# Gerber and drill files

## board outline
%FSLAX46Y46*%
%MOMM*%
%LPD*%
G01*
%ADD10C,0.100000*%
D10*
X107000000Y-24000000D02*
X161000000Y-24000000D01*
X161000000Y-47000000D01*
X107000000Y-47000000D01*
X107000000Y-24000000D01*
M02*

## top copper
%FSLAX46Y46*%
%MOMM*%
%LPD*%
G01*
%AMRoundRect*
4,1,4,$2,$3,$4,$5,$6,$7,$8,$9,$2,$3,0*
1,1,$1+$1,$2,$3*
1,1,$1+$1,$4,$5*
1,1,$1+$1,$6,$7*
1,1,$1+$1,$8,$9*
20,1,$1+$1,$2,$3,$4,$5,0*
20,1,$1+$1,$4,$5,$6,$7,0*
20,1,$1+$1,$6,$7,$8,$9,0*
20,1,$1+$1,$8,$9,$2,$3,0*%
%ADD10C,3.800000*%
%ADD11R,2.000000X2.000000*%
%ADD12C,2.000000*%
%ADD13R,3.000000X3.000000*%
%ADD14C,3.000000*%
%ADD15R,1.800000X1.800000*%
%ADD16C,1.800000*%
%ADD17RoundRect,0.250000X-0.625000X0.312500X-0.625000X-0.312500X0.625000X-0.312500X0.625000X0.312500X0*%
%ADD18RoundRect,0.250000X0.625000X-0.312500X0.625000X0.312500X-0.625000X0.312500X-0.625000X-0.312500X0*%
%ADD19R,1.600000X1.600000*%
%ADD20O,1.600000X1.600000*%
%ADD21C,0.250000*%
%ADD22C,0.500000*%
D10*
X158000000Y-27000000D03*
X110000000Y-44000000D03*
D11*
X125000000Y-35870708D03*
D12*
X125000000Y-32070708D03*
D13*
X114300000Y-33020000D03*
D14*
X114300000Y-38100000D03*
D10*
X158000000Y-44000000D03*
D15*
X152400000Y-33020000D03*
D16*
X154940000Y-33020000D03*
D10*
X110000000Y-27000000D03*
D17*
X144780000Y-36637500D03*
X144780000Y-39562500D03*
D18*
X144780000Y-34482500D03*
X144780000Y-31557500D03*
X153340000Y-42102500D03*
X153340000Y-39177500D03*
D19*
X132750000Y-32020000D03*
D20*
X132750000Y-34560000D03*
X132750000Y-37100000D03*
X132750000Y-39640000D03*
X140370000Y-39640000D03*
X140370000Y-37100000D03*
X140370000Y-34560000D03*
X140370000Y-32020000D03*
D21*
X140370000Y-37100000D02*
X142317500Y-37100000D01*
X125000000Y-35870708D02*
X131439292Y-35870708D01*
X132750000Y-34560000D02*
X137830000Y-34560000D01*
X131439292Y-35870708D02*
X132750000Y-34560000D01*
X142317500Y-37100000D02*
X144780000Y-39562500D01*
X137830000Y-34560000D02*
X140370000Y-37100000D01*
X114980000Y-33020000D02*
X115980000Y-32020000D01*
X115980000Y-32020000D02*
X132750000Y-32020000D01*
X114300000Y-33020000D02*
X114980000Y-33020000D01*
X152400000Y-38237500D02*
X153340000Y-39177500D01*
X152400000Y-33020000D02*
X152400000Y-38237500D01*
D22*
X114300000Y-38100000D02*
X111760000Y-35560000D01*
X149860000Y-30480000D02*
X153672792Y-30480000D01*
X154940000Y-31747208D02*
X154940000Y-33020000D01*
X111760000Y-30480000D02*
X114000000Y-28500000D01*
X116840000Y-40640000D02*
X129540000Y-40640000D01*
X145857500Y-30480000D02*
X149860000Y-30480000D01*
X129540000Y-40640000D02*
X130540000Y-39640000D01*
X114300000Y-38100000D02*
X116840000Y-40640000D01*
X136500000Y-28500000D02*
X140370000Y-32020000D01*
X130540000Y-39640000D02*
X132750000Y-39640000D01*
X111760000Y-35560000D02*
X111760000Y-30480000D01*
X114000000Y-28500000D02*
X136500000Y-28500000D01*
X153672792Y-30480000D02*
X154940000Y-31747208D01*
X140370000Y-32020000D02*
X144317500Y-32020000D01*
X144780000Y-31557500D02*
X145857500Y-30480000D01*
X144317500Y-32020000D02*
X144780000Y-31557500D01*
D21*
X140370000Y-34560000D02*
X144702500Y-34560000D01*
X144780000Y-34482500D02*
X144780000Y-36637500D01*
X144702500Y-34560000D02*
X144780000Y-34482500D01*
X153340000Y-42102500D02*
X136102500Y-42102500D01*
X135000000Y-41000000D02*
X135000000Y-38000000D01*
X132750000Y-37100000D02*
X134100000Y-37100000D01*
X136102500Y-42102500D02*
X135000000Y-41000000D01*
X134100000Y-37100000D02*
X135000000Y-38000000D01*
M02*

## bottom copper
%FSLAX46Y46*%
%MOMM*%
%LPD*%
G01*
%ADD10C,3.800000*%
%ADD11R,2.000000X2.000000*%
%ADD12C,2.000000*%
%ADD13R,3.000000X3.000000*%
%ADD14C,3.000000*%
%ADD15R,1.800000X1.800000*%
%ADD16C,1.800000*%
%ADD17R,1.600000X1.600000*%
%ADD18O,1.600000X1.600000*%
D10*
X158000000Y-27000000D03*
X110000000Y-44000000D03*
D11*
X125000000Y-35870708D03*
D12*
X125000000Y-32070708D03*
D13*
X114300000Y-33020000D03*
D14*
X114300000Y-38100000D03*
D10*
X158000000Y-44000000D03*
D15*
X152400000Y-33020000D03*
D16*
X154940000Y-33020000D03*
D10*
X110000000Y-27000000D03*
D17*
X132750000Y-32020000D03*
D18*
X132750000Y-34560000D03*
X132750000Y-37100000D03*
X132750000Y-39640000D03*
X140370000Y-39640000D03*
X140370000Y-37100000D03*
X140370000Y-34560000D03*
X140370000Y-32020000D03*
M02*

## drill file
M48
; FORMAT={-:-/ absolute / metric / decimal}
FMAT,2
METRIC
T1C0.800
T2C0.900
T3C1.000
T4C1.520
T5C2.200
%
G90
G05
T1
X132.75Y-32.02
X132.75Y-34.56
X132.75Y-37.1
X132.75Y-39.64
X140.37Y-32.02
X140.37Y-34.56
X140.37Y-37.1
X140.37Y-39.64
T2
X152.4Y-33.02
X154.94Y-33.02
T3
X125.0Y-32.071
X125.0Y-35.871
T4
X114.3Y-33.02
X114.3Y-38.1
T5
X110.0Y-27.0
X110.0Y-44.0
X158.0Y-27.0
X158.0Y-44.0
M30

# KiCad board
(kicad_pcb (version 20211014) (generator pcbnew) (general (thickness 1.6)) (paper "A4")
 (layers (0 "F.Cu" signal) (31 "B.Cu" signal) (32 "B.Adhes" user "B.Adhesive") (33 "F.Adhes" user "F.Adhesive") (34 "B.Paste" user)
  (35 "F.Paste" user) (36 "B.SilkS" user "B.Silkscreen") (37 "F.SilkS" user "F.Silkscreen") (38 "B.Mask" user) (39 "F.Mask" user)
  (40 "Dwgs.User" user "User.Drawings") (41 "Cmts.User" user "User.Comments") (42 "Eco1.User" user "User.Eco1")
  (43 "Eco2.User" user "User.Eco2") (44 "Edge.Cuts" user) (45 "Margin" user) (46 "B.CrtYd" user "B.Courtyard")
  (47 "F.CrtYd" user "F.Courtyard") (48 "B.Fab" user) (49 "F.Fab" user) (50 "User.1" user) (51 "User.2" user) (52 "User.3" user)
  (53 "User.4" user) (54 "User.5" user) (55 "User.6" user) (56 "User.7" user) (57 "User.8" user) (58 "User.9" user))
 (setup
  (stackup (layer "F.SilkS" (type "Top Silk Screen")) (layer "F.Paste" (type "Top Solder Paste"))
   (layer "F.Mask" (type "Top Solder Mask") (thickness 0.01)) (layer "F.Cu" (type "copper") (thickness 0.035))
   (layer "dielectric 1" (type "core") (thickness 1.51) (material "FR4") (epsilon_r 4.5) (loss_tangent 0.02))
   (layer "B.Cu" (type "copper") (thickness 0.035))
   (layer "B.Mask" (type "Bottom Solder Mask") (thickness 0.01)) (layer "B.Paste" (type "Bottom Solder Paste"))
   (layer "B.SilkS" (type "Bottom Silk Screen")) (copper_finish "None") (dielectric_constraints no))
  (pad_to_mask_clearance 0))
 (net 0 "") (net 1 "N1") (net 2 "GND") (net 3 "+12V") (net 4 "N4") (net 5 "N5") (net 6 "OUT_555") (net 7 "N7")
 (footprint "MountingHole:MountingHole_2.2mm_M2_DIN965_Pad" (layer "F.Cu") (at 158 27)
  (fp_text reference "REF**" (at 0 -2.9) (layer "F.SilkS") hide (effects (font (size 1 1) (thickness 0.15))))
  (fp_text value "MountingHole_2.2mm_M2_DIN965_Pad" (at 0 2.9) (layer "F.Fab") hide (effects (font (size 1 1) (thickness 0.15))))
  (pad "1" thru_hole circle (at 0 0) (size 3.8 3.8) (drill 2.2) (layers *.Cu *.Mask)))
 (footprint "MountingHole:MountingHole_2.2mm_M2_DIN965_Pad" (layer "F.Cu") (at 110 44)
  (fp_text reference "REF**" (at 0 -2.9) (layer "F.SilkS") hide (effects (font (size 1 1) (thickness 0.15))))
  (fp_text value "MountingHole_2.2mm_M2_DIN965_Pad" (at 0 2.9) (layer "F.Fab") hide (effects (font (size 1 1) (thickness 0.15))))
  (pad "1" thru_hole circle (at 0 0) (size 3.8 3.8) (drill 2.2) (layers *.Cu *.Mask)))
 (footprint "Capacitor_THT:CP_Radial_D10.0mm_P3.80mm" (layer "F.Cu") (at 125 35.870708 90)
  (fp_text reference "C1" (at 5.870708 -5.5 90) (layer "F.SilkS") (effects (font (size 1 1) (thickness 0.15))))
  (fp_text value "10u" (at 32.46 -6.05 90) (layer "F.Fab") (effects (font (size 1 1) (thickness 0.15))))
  (pad "1" thru_hole rect (at 0 0 90) (size 2 2) (drill 1) (layers *.Cu *.Mask) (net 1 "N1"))
  (pad "2" thru_hole circle (at 3.8 0 90) (size 2 2) (drill 1) (layers *.Cu *.Mask) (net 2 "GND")))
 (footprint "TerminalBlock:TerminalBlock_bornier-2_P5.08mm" (layer "F.Cu") (at 114.3 33.02 -90)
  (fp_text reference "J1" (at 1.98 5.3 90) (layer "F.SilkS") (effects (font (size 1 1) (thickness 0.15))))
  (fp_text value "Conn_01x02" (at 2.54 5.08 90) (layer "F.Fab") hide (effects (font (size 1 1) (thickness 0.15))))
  (pad "1" thru_hole rect (at 0 0 270) (size 3 3) (drill 1.52) (layers *.Cu *.Mask) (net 2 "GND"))
  (pad "2" thru_hole circle (at 5.08 0 270) (size 3 3) (drill 1.52) (layers *.Cu *.Mask) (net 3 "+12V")))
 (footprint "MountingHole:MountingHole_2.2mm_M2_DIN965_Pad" (layer "F.Cu") (at 158 44)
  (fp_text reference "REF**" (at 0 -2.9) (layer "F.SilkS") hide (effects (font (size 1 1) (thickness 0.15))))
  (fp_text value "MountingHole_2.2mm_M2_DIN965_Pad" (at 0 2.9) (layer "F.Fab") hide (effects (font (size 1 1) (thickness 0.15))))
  (pad "1" thru_hole circle (at 0 0) (size 3.8 3.8) (drill 2.2) (layers *.Cu *.Mask)))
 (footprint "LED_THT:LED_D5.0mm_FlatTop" (layer "F.Cu") (at 152.4 33.02)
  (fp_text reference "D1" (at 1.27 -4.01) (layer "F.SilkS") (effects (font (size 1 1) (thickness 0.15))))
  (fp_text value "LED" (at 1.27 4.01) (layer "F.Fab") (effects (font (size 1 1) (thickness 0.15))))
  (pad "1" thru_hole rect locked (at 0 0) (size 1.8 1.8) (drill 0.9) (layers *.Cu *.Mask) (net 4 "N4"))
  (pad "2" thru_hole circle (at 2.54 0) (size 1.8 1.8) (drill 0.9) (layers *.Cu *.Mask) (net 3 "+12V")))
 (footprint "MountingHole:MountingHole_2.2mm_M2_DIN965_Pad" (layer "F.Cu") (at 110 27)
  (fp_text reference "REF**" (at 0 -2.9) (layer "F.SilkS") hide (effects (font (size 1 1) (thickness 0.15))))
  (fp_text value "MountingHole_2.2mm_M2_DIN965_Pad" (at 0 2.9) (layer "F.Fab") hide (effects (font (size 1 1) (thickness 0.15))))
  (pad "1" thru_hole circle (at 0 0) (size 3.8 3.8) (drill 2.2) (layers *.Cu *.Mask)))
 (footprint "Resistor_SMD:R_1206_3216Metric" (layer "F.Cu") (at 144.78 38.1 -90)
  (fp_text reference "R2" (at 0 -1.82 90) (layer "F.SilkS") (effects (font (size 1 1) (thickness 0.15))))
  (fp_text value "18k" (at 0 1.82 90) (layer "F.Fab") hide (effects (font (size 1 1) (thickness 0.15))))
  (pad "1" smd roundrect (at -1.4625 0 270) (size 1.125 1.75) (layers "F.Cu" "F.Paste" "F.Mask") (roundrect_rratio 0.222222) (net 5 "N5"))
  (pad "2" smd roundrect (at 1.4625 0 270) (size 1.125 1.75) (layers "F.Cu" "F.Paste" "F.Mask") (roundrect_rratio 0.222222) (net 1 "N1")))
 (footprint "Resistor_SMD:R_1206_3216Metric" (layer "F.Cu") (at 144.78 33.02 90)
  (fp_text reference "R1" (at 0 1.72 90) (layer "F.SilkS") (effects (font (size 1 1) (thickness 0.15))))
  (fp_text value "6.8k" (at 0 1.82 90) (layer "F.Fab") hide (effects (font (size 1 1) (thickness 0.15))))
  (pad "1" smd roundrect (at -1.4625 0 90) (size 1.125 1.75) (layers "F.Cu" "F.Paste" "F.Mask") (roundrect_rratio 0.222222) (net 5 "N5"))
  (pad "2" smd roundrect (at 1.4625 0 90) (size 1.125 1.75) (layers "F.Cu" "F.Paste" "F.Mask") (roundrect_rratio 0.222222) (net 3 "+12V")))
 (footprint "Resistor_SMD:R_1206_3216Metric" (layer "F.Cu") (at 153.34 40.64 90)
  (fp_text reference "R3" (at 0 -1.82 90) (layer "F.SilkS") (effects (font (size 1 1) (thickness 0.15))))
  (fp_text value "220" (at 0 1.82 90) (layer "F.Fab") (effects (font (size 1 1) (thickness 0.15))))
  (pad "1" smd roundrect (at -1.4625 0 90) (size 1.125 1.75) (layers "F.Cu" "F.Paste" "F.Mask") (roundrect_rratio 0.222222)
   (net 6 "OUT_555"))
  (pad "2" smd roundrect (at 1.4625 0 90) (size 1.125 1.75) (layers "F.Cu" "F.Paste" "F.Mask") (roundrect_rratio 0.222222) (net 4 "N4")))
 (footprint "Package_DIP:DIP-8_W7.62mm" (layer "F.Cu") (at 132.75 32.02)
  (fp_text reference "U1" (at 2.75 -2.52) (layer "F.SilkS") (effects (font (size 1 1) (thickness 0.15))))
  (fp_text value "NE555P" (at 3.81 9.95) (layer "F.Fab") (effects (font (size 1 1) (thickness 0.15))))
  (pad "1" thru_hole rect (at 0 0) (size 1.6 1.6) (drill 0.8) (layers *.Cu *.Mask) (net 2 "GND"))
  (pad "2" thru_hole oval (at 0 2.54) (size 1.6 1.6) (drill 0.8) (layers *.Cu *.Mask) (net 1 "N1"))
  (pad "3" thru_hole oval (at 0 5.08) (size 1.6 1.6) (drill 0.8) (layers *.Cu *.Mask) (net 6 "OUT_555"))
  (pad "4" thru_hole oval (at 0 7.62) (size 1.6 1.6) (drill 0.8) (layers *.Cu *.Mask) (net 3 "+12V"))
  (pad "5" thru_hole oval (at 7.62 7.62) (size 1.6 1.6) (drill 0.8) (layers *.Cu *.Mask) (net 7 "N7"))
  (pad "6" thru_hole oval (at 7.62 5.08) (size 1.6 1.6) (drill 0.8) (layers *.Cu *.Mask) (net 1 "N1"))
  (pad "7" thru_hole oval (at 7.62 2.54) (size 1.6 1.6) (drill 0.8) (layers *.Cu *.Mask) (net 5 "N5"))
  (pad "8" thru_hole oval (at 7.62 0) (size 1.6 1.6) (drill 0.8) (layers *.Cu *.Mask) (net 3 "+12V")))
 (gr_rect (start 107 24) (end 161 47) (layer "Edge.Cuts") (width 0.1) (fill none))
 (segment (start 140.37 37.1) (end 142.3175 37.1) (width 0.25) (layer "F.Cu") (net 1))
 (segment (start 125 35.870708) (end 131.439292 35.870708) (width 0.25) (layer "F.Cu") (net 1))
 (segment (start 132.75 34.56) (end 137.83 34.56) (width 0.25) (layer "F.Cu") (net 1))
 (segment (start 131.439292 35.870708) (end 132.75 34.56) (width 0.25) (layer "F.Cu") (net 1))
 (segment (start 142.3175 37.1) (end 144.78 39.5625) (width 0.25) (layer "F.Cu") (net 1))
 (segment (start 137.83 34.56) (end 140.37 37.1) (width 0.25) (layer "F.Cu") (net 1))
 (segment (start 114.98 33.02) (end 115.98 32.02) (width 0.25) (layer "F.Cu") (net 2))
 (segment (start 115.98 32.02) (end 132.75 32.02) (width 0.25) (layer "F.Cu") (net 2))
 (segment (start 114.3 33.02) (end 114.98 33.02) (width 0.25) (layer "F.Cu") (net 2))
 (segment (start 152.4 38.2375) (end 153.34 39.1775) (width 0.25) (layer "F.Cu") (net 4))
 (segment (start 152.4 33.02) (end 152.4 38.2375) (width 0.25) (layer "F.Cu") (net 4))
 (segment (start 114.3 38.1) (end 111.76 35.56) (width 0.5) (layer "F.Cu") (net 3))
 (segment (start 149.86 30.48) (end 153.672792 30.48) (width 0.5) (layer "F.Cu") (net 3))
 (segment (start 154.94 31.747208) (end 154.94 33.02) (width 0.5) (layer "F.Cu") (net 3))
 (segment (start 111.76 30.48) (end 114 28.5) (width 0.5) (layer "F.Cu") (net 3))
 (segment (start 116.84 40.64) (end 129.54 40.64) (width 0.5) (layer "F.Cu") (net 3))
 (segment (start 145.8575 30.48) (end 149.86 30.48) (width 0.5) (layer "F.Cu") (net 3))
 (segment (start 129.54 40.64) (end 130.54 39.64) (width 0.5) (layer "F.Cu") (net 3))
 (segment (start 114.3 38.1) (end 116.84 40.64) (width 0.5) (layer "F.Cu") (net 3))
 (segment (start 136.5 28.5) (end 140.37 32.02) (width 0.5) (layer "F.Cu") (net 3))
 (segment (start 130.54 39.64) (end 132.75 39.64) (width 0.5) (layer "F.Cu") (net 3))
 (segment (start 111.76 35.56) (end 111.76 30.48) (width 0.5) (layer "F.Cu") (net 3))
 (segment (start 114 28.5) (end 136.5 28.5) (width 0.5) (layer "F.Cu") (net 3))
 (segment (start 153.672792 30.48) (end 154.94 31.747208) (width 0.5) (layer "F.Cu") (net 3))
 (segment (start 140.37 32.02) (end 144.3175 32.02) (width 0.5) (layer "F.Cu") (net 3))
 (segment (start 144.78 31.5575) (end 145.8575 30.48) (width 0.5) (layer "F.Cu") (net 3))
 (segment (start 144.3175 32.02) (end 144.78 31.5575) (width 0.5) (layer "F.Cu") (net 3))
 (segment (start 140.37 34.56) (end 144.7025 34.56) (width 0.25) (layer "F.Cu") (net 5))
 (segment (start 144.78 34.4825) (end 144.78 36.6375) (width 0.25) (layer "F.Cu") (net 5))
 (segment (start 144.7025 34.56) (end 144.78 34.4825) (width 0.25) (layer "F.Cu") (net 5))
 (segment (start 153.34 42.1025) (end 136.1025 42.1025) (width 0.25) (layer "F.Cu") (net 6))
 (segment (start 135 41) (end 135 38) (width 0.25) (layer "F.Cu") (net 6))
 (segment (start 132.75 37.1) (end 134.1 37.1) (width 0.25) (layer "F.Cu") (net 6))
 (segment (start 136.1025 42.1025) (end 135 41) (width 0.25) (layer "F.Cu") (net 6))
 (segment (start 134.1 37.1) (end 135 38) (width 0.25) (layer "F.Cu") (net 6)))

